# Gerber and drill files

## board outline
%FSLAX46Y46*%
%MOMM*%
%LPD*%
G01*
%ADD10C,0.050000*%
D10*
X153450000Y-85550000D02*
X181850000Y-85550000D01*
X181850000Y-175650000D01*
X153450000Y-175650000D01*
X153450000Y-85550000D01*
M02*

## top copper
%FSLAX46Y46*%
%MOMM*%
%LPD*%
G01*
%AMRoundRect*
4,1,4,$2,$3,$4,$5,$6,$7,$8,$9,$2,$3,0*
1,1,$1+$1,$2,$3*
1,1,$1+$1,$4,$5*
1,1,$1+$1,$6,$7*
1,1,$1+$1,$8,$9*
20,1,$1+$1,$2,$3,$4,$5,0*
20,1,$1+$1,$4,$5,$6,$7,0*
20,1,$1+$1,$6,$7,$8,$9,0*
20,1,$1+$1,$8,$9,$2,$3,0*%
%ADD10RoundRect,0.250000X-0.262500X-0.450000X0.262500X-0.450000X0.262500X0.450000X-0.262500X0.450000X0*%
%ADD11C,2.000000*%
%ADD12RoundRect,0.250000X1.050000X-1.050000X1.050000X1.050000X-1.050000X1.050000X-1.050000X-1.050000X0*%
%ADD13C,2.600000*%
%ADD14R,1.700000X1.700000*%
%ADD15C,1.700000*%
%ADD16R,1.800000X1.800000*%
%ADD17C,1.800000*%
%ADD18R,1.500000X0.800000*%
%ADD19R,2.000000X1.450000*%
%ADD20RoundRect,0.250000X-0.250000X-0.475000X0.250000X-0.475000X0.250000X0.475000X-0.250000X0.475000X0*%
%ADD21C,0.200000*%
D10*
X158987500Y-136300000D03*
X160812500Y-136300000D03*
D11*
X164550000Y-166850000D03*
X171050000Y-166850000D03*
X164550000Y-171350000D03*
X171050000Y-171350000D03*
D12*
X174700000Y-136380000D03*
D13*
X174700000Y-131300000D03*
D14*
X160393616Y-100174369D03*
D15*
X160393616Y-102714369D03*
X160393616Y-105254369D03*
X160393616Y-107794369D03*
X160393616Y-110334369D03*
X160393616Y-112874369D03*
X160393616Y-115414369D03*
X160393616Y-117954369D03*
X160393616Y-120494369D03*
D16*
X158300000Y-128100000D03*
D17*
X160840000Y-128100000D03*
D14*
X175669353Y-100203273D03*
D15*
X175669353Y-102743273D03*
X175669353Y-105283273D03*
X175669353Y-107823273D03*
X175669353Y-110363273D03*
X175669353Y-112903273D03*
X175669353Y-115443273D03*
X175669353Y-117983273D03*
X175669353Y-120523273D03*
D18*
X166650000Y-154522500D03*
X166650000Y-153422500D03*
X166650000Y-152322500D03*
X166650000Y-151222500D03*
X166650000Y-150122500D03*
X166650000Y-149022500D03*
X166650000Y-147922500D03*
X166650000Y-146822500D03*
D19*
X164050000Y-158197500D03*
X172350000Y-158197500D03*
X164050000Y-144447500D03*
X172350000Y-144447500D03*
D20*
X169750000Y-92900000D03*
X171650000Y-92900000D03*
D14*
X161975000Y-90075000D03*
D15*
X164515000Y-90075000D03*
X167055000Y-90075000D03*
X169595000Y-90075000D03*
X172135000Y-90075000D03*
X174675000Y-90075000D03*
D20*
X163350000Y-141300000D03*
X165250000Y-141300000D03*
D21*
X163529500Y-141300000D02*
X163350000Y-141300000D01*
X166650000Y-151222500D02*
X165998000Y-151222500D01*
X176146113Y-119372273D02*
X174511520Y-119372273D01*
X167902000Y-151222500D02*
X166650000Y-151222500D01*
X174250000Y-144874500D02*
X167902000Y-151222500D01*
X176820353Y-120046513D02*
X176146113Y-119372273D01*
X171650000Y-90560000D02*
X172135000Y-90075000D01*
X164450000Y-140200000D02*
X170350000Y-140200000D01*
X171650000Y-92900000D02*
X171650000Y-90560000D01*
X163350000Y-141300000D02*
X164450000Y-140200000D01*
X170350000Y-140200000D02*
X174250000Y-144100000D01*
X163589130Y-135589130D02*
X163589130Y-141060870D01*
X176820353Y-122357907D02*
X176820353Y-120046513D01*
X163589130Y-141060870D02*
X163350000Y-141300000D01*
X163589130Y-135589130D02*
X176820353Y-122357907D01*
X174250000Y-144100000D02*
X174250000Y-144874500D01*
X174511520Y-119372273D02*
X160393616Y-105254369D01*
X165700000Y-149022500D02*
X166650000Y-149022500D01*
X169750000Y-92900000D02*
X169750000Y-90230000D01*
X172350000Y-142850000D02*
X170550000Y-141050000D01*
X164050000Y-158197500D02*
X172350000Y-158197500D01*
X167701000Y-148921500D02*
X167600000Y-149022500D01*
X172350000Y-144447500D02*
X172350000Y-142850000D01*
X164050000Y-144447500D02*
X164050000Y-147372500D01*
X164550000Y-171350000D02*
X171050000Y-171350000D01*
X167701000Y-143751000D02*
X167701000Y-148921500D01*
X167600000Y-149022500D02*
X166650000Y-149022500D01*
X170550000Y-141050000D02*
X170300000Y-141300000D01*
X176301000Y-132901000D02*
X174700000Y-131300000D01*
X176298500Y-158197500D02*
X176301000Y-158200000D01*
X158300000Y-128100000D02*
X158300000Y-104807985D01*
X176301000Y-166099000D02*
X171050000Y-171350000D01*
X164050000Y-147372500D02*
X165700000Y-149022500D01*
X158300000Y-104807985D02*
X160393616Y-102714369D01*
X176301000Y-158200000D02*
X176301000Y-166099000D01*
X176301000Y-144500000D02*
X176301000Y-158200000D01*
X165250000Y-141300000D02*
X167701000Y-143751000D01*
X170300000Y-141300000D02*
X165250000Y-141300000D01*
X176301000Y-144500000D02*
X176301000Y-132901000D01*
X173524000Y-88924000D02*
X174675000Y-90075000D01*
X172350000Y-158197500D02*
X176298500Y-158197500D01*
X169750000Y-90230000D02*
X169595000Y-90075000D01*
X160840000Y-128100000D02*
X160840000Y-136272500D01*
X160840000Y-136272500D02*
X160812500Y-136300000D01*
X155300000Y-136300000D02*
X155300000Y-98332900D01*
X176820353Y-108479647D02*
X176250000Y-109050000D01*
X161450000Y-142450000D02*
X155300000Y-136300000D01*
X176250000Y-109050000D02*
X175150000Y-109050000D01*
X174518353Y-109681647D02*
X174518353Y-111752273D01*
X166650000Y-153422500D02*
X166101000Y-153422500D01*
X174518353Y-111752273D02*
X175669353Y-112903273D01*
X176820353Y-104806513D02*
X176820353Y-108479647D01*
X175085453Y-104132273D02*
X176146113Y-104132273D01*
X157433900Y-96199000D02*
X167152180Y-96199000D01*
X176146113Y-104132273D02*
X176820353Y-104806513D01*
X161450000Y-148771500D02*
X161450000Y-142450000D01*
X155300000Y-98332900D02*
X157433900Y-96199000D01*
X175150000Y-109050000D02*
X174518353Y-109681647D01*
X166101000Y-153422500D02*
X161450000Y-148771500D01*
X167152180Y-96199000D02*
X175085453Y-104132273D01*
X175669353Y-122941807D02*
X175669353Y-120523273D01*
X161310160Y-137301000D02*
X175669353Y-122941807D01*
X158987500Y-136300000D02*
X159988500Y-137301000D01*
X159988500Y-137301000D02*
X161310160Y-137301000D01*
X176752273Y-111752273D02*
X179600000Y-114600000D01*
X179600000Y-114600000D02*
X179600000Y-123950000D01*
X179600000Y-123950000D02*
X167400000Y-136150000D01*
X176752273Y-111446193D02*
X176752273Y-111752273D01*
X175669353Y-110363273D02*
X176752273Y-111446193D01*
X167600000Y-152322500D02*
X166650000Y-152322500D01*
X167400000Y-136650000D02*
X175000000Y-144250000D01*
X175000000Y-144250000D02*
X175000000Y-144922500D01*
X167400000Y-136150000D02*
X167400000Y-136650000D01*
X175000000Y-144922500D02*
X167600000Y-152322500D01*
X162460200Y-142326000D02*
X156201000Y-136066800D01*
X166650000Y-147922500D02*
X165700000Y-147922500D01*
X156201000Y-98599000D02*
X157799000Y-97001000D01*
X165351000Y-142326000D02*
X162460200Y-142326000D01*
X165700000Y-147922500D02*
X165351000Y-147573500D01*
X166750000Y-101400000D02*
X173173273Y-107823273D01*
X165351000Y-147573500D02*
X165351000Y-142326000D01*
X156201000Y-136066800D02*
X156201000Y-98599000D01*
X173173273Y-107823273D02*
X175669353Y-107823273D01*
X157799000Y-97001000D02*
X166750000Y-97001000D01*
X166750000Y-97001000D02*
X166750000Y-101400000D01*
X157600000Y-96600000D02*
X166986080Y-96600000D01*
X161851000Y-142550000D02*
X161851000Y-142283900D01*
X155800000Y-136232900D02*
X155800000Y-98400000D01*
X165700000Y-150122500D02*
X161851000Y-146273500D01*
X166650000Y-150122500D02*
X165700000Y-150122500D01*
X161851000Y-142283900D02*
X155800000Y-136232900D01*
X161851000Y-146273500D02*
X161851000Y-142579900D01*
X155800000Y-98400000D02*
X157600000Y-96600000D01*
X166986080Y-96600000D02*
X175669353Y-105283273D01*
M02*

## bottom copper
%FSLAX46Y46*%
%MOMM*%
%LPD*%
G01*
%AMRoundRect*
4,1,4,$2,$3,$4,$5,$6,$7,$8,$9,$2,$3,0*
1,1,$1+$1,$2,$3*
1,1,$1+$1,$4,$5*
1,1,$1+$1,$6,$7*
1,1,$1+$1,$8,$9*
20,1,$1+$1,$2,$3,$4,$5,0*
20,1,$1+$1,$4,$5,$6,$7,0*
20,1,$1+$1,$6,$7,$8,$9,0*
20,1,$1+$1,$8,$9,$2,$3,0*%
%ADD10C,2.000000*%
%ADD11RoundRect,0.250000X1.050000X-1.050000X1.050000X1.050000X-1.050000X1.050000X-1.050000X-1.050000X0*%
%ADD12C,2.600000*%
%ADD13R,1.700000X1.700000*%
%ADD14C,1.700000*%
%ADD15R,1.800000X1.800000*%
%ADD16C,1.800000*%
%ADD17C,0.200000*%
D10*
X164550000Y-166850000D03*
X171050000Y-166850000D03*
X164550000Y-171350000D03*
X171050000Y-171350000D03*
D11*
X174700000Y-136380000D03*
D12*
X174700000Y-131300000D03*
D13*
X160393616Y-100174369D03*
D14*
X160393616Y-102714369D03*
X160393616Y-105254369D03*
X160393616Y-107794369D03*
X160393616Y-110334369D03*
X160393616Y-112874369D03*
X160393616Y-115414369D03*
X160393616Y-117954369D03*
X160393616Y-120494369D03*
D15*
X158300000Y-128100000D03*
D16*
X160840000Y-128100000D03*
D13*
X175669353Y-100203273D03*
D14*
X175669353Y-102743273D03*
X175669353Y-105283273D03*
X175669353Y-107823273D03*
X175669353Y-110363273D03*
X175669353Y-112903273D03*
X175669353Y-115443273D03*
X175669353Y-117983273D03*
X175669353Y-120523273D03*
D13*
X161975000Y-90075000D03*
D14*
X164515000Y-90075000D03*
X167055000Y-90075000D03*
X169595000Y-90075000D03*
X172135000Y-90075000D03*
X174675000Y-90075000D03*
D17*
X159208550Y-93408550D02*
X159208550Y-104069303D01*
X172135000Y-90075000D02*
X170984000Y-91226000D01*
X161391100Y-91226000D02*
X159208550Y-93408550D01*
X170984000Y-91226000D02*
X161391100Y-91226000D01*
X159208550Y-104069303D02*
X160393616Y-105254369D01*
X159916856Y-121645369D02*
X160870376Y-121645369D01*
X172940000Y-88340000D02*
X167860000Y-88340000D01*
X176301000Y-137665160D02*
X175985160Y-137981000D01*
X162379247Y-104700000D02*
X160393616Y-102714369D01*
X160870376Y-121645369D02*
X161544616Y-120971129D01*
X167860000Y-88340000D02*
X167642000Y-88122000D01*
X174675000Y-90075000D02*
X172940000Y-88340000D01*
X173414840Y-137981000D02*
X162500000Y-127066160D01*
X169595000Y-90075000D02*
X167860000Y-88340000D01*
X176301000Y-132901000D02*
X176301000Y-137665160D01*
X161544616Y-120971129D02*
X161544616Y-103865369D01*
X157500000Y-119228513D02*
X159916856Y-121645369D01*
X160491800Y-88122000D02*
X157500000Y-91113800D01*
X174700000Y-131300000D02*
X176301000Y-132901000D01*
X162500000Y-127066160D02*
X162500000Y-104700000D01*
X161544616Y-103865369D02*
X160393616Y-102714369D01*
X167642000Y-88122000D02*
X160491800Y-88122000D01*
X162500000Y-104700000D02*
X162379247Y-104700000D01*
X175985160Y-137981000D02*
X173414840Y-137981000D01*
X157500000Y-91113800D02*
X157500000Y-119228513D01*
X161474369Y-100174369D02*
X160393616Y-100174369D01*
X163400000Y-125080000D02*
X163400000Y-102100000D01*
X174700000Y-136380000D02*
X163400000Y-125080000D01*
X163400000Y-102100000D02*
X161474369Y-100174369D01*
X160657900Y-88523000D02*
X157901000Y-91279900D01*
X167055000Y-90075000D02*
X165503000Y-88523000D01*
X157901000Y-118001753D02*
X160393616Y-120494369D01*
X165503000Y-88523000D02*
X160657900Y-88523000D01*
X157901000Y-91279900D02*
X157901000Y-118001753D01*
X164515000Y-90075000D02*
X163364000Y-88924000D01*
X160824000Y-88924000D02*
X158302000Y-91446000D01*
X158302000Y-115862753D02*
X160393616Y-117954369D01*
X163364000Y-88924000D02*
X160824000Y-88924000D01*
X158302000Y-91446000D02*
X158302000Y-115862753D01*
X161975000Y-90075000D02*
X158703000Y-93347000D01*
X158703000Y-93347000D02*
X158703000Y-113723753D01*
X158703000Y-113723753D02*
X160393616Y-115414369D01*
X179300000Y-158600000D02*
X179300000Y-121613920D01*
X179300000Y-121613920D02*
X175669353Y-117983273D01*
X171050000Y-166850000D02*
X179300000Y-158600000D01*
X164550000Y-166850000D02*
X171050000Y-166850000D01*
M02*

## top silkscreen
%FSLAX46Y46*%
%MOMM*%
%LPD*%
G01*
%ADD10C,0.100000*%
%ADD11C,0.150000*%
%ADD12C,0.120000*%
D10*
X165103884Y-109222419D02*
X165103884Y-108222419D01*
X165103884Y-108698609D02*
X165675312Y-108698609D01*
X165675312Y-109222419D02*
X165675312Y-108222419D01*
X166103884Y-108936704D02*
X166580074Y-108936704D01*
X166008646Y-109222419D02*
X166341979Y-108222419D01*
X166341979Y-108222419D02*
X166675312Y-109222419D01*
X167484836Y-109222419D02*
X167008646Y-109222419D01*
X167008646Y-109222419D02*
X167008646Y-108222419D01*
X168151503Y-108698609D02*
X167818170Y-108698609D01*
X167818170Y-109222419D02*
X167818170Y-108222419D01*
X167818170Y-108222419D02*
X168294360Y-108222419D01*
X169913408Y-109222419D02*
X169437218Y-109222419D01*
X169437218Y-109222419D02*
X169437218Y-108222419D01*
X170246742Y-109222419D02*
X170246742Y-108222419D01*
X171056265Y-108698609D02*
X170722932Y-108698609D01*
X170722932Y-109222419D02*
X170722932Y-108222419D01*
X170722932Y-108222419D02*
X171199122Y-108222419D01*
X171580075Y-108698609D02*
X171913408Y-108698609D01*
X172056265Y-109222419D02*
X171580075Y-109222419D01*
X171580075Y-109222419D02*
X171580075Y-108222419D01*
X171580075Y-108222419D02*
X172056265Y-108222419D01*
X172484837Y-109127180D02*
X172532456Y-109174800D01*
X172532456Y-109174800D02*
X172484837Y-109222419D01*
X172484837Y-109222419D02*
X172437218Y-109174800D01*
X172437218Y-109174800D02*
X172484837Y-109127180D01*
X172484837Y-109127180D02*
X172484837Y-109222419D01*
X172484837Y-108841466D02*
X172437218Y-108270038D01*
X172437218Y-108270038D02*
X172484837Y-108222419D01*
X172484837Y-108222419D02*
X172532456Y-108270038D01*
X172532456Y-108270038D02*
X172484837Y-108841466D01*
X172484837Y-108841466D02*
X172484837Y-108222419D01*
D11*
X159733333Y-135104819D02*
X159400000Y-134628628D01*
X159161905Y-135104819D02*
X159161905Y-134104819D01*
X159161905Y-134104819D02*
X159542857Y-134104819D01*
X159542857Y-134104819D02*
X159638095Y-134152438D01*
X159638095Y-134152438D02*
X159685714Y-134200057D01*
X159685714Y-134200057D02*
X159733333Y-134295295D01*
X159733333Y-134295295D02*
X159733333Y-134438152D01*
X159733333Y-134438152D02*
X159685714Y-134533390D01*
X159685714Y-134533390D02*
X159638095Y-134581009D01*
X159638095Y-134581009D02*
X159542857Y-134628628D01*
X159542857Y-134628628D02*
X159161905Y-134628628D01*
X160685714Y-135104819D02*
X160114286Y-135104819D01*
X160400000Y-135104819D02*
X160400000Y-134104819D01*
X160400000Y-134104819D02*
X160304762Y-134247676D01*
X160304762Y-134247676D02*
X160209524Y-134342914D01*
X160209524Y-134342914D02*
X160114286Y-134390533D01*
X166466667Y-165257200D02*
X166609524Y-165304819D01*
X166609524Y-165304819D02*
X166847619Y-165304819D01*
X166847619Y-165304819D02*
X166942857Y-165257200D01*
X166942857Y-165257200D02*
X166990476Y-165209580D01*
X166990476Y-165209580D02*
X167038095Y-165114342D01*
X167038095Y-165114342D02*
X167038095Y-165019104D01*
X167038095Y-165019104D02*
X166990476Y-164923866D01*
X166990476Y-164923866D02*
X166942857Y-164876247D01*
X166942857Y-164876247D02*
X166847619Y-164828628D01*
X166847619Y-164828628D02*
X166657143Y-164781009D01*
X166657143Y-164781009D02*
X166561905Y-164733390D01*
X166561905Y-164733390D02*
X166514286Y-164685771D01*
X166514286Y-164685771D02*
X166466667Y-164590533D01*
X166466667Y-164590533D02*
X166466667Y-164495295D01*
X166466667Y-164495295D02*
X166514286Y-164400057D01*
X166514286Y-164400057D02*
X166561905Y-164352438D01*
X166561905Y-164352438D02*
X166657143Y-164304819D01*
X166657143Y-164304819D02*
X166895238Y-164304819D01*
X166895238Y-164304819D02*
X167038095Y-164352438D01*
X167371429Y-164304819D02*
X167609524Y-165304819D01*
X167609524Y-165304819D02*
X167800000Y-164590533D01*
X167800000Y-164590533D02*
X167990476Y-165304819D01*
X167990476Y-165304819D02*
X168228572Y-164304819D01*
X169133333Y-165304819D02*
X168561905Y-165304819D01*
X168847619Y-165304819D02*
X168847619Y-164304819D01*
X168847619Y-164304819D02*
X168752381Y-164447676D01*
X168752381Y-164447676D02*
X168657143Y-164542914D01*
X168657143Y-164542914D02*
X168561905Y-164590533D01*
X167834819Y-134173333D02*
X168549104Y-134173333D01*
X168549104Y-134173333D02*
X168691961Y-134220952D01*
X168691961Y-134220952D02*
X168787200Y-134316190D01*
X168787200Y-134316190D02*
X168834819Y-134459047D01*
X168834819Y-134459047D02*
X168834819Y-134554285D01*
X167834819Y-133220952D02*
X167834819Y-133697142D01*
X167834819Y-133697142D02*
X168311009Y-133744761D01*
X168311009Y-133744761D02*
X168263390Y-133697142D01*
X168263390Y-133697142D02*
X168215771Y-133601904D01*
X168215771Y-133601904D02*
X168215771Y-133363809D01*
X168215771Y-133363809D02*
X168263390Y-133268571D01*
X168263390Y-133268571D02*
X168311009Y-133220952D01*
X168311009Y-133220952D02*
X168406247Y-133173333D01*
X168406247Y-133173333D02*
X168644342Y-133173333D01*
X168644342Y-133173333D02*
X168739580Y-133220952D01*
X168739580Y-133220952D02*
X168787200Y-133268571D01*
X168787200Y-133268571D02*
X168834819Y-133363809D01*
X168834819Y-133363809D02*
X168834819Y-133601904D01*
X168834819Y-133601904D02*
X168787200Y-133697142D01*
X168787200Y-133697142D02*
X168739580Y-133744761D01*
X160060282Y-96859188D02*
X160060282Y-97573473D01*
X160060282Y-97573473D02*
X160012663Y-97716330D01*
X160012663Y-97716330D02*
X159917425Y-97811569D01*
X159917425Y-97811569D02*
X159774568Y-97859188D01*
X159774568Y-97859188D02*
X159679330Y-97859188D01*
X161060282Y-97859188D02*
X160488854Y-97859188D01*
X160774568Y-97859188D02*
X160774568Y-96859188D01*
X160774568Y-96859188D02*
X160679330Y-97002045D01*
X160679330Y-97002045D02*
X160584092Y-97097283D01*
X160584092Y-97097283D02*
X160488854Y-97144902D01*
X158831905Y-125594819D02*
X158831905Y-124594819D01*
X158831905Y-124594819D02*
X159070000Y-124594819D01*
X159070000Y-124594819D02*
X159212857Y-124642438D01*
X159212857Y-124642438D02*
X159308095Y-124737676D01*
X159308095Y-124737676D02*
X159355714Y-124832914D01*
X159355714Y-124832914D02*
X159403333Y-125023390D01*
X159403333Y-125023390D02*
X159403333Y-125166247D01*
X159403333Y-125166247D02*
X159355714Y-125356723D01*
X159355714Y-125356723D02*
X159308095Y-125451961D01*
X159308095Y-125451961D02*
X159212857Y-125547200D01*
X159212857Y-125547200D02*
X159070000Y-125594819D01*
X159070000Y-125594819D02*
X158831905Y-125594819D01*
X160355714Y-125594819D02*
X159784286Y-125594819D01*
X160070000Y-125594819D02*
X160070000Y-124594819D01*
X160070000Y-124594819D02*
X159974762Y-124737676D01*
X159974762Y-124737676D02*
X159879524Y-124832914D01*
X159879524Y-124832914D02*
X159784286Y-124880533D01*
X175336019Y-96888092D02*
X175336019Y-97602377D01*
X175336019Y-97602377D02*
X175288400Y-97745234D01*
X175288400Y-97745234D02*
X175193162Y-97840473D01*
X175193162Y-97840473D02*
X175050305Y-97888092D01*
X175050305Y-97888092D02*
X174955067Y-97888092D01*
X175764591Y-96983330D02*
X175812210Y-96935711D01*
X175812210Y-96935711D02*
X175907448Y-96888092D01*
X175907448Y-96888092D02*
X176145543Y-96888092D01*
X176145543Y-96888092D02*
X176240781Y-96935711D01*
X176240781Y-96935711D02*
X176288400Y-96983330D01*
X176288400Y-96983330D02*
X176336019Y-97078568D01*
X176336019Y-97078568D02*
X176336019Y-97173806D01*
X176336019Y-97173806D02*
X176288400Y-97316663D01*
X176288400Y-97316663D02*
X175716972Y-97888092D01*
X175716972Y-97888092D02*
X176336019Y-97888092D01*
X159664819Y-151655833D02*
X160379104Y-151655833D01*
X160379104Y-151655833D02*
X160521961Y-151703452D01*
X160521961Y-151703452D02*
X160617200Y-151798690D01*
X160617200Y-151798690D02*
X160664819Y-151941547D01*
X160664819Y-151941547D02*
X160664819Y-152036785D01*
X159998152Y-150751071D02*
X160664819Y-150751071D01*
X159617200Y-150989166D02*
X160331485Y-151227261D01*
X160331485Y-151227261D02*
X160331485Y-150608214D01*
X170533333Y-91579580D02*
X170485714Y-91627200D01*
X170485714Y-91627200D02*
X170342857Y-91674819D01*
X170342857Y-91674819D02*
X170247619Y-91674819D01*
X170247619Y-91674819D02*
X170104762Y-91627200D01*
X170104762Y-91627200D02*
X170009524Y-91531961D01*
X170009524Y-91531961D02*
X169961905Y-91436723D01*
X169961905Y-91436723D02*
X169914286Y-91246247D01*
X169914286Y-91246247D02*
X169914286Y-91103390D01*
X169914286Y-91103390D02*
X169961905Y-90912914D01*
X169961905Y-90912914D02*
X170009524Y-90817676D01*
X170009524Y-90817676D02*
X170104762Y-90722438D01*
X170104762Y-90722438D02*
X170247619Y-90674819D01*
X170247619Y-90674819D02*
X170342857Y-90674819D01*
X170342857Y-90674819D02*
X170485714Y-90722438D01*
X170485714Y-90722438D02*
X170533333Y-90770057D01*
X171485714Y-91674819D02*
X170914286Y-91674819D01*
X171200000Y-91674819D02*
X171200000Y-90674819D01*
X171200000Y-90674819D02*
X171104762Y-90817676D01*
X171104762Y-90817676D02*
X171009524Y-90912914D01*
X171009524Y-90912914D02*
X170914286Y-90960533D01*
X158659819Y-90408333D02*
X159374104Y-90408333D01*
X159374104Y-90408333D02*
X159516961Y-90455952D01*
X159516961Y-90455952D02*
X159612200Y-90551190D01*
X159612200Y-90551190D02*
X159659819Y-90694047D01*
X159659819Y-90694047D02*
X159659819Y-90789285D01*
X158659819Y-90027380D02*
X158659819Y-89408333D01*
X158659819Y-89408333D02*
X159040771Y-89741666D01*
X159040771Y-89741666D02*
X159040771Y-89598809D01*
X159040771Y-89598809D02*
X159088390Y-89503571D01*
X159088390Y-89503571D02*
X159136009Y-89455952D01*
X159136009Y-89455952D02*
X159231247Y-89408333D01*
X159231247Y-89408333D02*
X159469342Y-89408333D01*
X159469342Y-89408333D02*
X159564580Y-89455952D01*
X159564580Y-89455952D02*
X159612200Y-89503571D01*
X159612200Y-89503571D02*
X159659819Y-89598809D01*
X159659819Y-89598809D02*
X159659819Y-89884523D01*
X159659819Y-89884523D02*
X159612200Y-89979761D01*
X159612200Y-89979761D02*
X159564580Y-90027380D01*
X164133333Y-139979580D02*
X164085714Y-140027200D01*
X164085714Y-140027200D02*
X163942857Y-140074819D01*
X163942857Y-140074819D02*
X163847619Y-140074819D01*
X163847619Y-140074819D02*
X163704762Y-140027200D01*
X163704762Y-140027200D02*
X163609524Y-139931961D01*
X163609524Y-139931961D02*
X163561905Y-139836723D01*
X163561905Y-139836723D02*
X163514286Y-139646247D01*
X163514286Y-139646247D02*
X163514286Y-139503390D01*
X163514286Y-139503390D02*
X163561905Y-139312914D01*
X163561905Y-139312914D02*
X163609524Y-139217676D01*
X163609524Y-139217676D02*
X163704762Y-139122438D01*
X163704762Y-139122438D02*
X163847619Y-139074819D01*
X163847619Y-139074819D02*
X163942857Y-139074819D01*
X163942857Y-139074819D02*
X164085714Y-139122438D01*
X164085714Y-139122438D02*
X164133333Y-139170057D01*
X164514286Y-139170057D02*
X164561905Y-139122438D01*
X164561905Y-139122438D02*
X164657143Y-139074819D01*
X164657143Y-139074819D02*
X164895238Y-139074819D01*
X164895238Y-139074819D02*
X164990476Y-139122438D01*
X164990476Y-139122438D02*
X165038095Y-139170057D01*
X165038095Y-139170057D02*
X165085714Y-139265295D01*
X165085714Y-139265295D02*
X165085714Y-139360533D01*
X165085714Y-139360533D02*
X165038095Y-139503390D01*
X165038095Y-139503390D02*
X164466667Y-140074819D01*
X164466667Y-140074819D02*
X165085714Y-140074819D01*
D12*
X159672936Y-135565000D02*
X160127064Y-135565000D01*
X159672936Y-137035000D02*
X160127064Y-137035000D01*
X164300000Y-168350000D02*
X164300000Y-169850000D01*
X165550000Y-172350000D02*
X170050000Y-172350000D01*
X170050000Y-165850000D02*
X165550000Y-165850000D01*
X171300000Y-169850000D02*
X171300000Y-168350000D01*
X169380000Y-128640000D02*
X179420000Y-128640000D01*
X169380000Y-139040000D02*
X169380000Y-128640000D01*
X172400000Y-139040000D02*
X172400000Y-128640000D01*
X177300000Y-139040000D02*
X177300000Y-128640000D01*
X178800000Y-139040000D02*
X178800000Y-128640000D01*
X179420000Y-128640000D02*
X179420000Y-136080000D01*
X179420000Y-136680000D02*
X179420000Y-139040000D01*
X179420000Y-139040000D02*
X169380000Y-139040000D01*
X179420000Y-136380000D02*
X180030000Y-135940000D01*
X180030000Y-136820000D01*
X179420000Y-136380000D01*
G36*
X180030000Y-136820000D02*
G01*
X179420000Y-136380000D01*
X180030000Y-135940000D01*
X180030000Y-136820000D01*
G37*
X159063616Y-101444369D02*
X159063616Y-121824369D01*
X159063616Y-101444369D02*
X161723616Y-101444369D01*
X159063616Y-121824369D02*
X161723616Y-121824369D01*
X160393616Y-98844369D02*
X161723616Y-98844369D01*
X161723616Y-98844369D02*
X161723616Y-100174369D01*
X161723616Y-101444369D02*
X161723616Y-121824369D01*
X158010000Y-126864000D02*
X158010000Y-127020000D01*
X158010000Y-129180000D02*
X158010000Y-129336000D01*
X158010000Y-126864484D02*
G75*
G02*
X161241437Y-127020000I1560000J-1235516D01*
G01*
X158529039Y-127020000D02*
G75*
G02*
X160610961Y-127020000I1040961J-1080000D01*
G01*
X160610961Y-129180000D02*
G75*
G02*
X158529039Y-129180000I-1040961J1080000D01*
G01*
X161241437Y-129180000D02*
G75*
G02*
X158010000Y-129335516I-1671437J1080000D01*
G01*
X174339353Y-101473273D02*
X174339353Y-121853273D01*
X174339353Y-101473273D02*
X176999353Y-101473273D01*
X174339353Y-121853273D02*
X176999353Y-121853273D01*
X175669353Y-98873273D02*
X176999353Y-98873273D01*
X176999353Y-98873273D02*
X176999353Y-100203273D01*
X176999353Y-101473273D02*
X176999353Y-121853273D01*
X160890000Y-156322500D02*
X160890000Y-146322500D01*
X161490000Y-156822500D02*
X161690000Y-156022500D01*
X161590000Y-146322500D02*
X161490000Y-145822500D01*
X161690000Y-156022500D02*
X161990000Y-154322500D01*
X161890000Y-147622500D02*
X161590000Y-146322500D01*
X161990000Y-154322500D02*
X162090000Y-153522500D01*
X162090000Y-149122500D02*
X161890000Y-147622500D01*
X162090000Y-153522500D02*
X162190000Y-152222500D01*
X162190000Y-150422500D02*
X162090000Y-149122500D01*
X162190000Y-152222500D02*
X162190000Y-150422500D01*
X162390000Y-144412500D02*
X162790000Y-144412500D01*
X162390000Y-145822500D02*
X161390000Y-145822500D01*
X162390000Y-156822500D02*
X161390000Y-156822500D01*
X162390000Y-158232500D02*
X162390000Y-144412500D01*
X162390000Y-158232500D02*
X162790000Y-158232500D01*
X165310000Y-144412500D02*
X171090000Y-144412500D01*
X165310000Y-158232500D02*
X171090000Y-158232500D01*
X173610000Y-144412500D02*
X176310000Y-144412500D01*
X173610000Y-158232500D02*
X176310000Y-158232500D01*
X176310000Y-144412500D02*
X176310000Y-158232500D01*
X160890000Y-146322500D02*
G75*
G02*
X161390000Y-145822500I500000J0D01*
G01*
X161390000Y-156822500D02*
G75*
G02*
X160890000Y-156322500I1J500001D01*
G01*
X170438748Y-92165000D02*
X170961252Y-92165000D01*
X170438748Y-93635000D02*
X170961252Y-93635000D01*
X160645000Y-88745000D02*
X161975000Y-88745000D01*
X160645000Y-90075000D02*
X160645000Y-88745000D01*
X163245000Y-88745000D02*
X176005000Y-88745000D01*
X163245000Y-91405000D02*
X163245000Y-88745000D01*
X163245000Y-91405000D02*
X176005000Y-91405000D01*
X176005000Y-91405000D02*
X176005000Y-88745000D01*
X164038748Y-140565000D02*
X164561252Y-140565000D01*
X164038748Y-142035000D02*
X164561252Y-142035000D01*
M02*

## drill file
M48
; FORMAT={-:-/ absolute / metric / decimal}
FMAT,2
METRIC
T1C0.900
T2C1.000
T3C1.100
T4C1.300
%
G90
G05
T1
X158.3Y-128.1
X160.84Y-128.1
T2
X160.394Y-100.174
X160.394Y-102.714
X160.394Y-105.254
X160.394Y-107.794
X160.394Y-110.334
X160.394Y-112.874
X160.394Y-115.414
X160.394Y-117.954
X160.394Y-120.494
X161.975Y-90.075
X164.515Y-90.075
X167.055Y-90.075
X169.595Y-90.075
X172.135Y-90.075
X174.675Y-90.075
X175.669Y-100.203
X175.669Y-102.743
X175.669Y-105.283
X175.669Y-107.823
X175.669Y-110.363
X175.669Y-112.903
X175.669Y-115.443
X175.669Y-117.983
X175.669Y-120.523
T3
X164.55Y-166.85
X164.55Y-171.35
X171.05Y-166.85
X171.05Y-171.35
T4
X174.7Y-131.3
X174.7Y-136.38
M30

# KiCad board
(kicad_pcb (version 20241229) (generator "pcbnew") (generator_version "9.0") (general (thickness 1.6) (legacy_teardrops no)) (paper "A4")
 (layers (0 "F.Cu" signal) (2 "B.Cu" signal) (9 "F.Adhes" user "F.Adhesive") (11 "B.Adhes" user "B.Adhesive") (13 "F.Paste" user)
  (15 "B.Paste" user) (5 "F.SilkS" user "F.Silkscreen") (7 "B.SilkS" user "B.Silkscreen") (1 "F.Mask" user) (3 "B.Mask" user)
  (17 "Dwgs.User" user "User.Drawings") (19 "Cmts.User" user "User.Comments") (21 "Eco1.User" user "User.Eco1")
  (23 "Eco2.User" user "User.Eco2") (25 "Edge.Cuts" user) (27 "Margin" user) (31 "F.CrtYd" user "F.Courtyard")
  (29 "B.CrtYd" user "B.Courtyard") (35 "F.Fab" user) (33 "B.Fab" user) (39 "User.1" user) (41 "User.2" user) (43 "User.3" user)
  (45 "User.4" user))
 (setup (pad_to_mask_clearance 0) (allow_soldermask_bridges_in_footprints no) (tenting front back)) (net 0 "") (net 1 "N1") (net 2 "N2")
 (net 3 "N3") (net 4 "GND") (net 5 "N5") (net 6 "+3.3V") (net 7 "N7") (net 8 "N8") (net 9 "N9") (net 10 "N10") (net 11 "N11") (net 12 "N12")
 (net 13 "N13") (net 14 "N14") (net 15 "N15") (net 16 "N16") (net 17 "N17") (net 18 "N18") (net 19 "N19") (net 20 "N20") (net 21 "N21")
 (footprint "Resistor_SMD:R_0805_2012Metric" (layer "F.Cu") (at 159.9 136.3)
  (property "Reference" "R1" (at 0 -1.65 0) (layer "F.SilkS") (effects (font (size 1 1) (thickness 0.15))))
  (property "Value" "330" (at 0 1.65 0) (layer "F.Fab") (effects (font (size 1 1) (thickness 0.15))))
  (fp_line (start -0.227064 -0.735) (end 0.227064 -0.735) (stroke (width 0.12) (type solid)) (layer "F.SilkS"))
  (fp_line (start -0.227064 0.735) (end 0.227064 0.735) (stroke (width 0.12) (type solid)) (layer "F.SilkS"))
  (pad "1" smd roundrect (at -0.9125 0) (size 1.025 1.4) (layers "F.Cu" "F.Mask" "F.Paste") (roundrect_rratio 0.243902) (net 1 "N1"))
  (pad "2" smd roundrect (at 0.9125 0) (size 1.025 1.4) (layers "F.Cu" "F.Mask" "F.Paste") (roundrect_rratio 0.243902) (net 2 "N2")))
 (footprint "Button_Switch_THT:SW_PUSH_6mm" (layer "F.Cu") (at 164.55 166.85)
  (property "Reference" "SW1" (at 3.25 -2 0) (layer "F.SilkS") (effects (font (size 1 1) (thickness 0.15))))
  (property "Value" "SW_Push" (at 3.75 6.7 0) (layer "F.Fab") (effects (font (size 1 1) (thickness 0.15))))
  (fp_line (start -0.25 1.5) (end -0.25 3) (stroke (width 0.12) (type solid)) (layer "F.SilkS"))
  (fp_line (start 1 5.5) (end 5.5 5.5) (stroke (width 0.12) (type solid)) (layer "F.SilkS"))
  (fp_line (start 5.5 -1) (end 1 -1) (stroke (width 0.12) (type solid)) (layer "F.SilkS"))
  (fp_line (start 6.75 3) (end 6.75 1.5) (stroke (width 0.12) (type solid)) (layer "F.SilkS"))
  (pad "1" thru_hole circle (at 0 0 90) (size 2 2) (drill 1.1) (layers "*.Cu" "*.Mask") (remove_unused_layers no) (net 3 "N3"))
  (pad "1" thru_hole circle (at 6.5 0 90) (size 2 2) (drill 1.1) (layers "*.Cu" "*.Mask") (remove_unused_layers no) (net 3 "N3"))
  (pad "2" thru_hole circle (at 0 4.5 90) (size 2 2) (drill 1.1) (layers "*.Cu" "*.Mask") (remove_unused_layers no) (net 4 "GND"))
  (pad "2" thru_hole circle (at 6.5 4.5 90) (size 2 2) (drill 1.1) (layers "*.Cu" "*.Mask") (remove_unused_layers no) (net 4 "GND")))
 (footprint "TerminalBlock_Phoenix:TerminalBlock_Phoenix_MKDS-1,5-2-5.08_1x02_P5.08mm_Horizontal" (layer "F.Cu") (at 174.7 136.38 90)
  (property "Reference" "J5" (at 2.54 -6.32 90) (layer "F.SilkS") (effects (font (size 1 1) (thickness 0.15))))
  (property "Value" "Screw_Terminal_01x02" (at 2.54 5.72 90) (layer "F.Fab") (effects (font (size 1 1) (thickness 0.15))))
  (fp_line (start 7.74 -5.32) (end 7.74 4.72) (stroke (width 0.12) (type solid)) (layer "F.SilkS"))
  (fp_line (start -2.66 -5.32) (end 7.74 -5.32) (stroke (width 0.12) (type solid)) (layer "F.SilkS"))
  (fp_line (start -2.66 -2.3) (end 7.74 -2.3) (stroke (width 0.12) (type solid)) (layer "F.SilkS"))
  (fp_line (start -2.66 2.6) (end 7.74 2.6) (stroke (width 0.12) (type solid)) (layer "F.SilkS"))
  (fp_line (start -2.66 4.1) (end 7.74 4.1) (stroke (width 0.12) (type solid)) (layer "F.SilkS"))
  (fp_line (start 7.74 4.72) (end 0.3 4.72) (stroke (width 0.12) (type solid)) (layer "F.SilkS"))
  (fp_line (start -0.3 4.72) (end -2.66 4.72) (stroke (width 0.12) (type solid)) (layer "F.SilkS"))
  (fp_line (start -2.66 4.72) (end -2.66 -5.32) (stroke (width 0.12) (type solid)) (layer "F.SilkS"))
  (fp_poly (pts (xy 0 4.72) (xy 0.44 5.33) (xy -0.44 5.33)) (stroke (width 0.12) (type solid)) (fill yes) (layer "F.SilkS"))
  (pad "1" thru_hole roundrect (at 0 0 90) (size 2.6 2.6) (drill 1.3) (layers "*.Cu" "*.Mask") (remove_unused_layers no)
   (roundrect_rratio 0.096154) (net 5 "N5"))
  (pad "2" thru_hole circle (at 5.08 0 90) (size 2.6 2.6) (drill 1.3) (layers "*.Cu" "*.Mask") (remove_unused_layers no) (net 4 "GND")))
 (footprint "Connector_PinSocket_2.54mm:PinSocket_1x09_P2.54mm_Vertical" (layer "F.Cu") (at 160.393616 100.174369)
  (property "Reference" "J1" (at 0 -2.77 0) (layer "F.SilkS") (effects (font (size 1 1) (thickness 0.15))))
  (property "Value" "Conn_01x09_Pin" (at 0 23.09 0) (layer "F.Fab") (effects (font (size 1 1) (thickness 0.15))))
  (fp_line (start -1.33 1.27) (end -1.33 21.65) (stroke (width 0.12) (type solid)) (layer "F.SilkS"))
  (fp_line (start -1.33 1.27) (end 1.33 1.27) (stroke (width 0.12) (type solid)) (layer "F.SilkS"))
  (fp_line (start -1.33 21.65) (end 1.33 21.65) (stroke (width 0.12) (type solid)) (layer "F.SilkS"))
  (fp_line (start 0 -1.33) (end 1.33 -1.33) (stroke (width 0.12) (type solid)) (layer "F.SilkS"))
  (fp_line (start 1.33 -1.33) (end 1.33 0) (stroke (width 0.12) (type solid)) (layer "F.SilkS"))
  (fp_line (start 1.33 1.27) (end 1.33 21.65) (stroke (width 0.12) (type solid)) (layer "F.SilkS"))
  (pad "1" thru_hole rect (at 0 0) (size 1.7 1.7) (drill 1) (layers "*.Cu" "*.Mask") (remove_unused_layers no) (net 5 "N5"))
  (pad "2" thru_hole circle (at 0 2.54) (size 1.7 1.7) (drill 1) (layers "*.Cu" "*.Mask") (remove_unused_layers no) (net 4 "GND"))
  (pad "3" thru_hole circle (at 0 5.08) (size 1.7 1.7) (drill 1) (layers "*.Cu" "*.Mask") (remove_unused_layers no) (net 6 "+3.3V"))
  (pad "4" thru_hole circle (at 0 7.62) (size 1.7 1.7) (drill 1) (layers "*.Cu" "*.Mask") (remove_unused_layers no) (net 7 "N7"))
  (pad "5" thru_hole circle (at 0 10.16) (size 1.7 1.7) (drill 1) (layers "*.Cu" "*.Mask") (remove_unused_layers no) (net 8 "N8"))
  (pad "6" thru_hole circle (at 0 12.7) (size 1.7 1.7) (drill 1) (layers "*.Cu" "*.Mask") (remove_unused_layers no) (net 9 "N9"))
  (pad "7" thru_hole circle (at 0 15.24) (size 1.7 1.7) (drill 1) (layers "*.Cu" "*.Mask") (remove_unused_layers no) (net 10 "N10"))
  (pad "8" thru_hole circle (at 0 17.78) (size 1.7 1.7) (drill 1) (layers "*.Cu" "*.Mask") (remove_unused_layers no) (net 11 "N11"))
  (pad "9" thru_hole circle (at 0 20.32) (size 1.7 1.7) (drill 1) (layers "*.Cu" "*.Mask") (remove_unused_layers no) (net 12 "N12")))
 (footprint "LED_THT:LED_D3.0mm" (layer "F.Cu") (at 158.3 128.1)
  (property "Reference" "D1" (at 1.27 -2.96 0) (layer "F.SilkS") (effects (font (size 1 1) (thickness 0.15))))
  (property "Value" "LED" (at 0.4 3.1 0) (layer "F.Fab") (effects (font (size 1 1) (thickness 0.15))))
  (fp_line (start -0.29 -1.236) (end -0.29 -1.08) (stroke (width 0.12) (type solid)) (layer "F.SilkS"))
  (fp_line (start -0.29 1.08) (end -0.29 1.236) (stroke (width 0.12) (type solid)) (layer "F.SilkS"))
  (fp_arc (start -0.29 -1.235516) (mid 1.36566 -1.987699) (end 2.941437 -1.08) (stroke (width 0.12) (type solid)) (layer "F.SilkS"))
  (fp_arc (start 0.229039 -1.08) (mid 1.27 -1.5) (end 2.310961 -1.08) (stroke (width 0.12) (type solid)) (layer "F.SilkS"))
  (fp_arc (start 2.310961 1.08) (mid 1.27 1.5) (end 0.229039 1.08) (stroke (width 0.12) (type solid)) (layer "F.SilkS"))
  (fp_arc (start 2.941437 1.08) (mid 1.36566 1.987699) (end -0.29 1.235516) (stroke (width 0.12) (type solid)) (layer "F.SilkS"))
  (pad "1" thru_hole rect (at 0 0) (size 1.8 1.8) (drill 0.9) (layers "*.Cu" "*.Mask") (remove_unused_layers no) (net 4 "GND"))
  (pad "2" thru_hole circle (at 2.54 0) (size 1.8 1.8) (drill 0.9) (layers "*.Cu" "*.Mask") (remove_unused_layers no) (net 2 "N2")))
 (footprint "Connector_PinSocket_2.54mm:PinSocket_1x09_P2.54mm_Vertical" (layer "F.Cu") (at 175.669353 100.203273)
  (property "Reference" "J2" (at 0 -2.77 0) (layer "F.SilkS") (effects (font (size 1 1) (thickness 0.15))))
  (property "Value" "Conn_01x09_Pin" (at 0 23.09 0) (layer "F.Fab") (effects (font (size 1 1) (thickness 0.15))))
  (fp_line (start -1.33 1.27) (end -1.33 21.65) (stroke (width 0.12) (type solid)) (layer "F.SilkS"))
  (fp_line (start -1.33 1.27) (end 1.33 1.27) (stroke (width 0.12) (type solid)) (layer "F.SilkS"))
  (fp_line (start -1.33 21.65) (end 1.33 21.65) (stroke (width 0.12) (type solid)) (layer "F.SilkS"))
  (fp_line (start 0 -1.33) (end 1.33 -1.33) (stroke (width 0.12) (type solid)) (layer "F.SilkS"))
  (fp_line (start 1.33 -1.33) (end 1.33 0) (stroke (width 0.12) (type solid)) (layer "F.SilkS"))
  (fp_line (start 1.33 1.27) (end 1.33 21.65) (stroke (width 0.12) (type solid)) (layer "F.SilkS"))
  (pad "1" thru_hole rect (at 0 0) (size 1.7 1.7) (drill 1) (layers "*.Cu" "*.Mask") (remove_unused_layers no) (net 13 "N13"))
  (pad "2" thru_hole circle (at 0 2.54) (size 1.7 1.7) (drill 1) (layers "*.Cu" "*.Mask") (remove_unused_layers no) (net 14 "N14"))
  (pad "3" thru_hole circle (at 0 5.08) (size 1.7 1.7) (drill 1) (layers "*.Cu" "*.Mask") (remove_unused_layers no) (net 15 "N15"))
  (pad "4" thru_hole circle (at 0 7.62) (size 1.7 1.7) (drill 1) (layers "*.Cu" "*.Mask") (remove_unused_layers no) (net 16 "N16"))
  (pad "5" thru_hole circle (at 0 10.16) (size 1.7 1.7) (drill 1) (layers "*.Cu" "*.Mask") (remove_unused_layers no) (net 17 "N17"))
  (pad "6" thru_hole circle (at 0 12.7) (size 1.7 1.7) (drill 1) (layers "*.Cu" "*.Mask") (remove_unused_layers no) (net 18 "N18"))
  (pad "7" thru_hole circle (at 0 15.24) (size 1.7 1.7) (drill 1) (layers "*.Cu" "*.Mask") (remove_unused_layers no) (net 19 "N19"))
  (pad "8" thru_hole circle (at 0 17.78) (size 1.7 1.7) (drill 1) (layers "*.Cu" "*.Mask") (remove_unused_layers no) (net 3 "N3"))
  (pad "9" thru_hole circle (at 0 20.32) (size 1.7 1.7) (drill 1) (layers "*.Cu" "*.Mask") (remove_unused_layers no) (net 1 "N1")))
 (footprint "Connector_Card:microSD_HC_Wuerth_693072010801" (layer "F.Cu") (at 168.2 151.3225 90)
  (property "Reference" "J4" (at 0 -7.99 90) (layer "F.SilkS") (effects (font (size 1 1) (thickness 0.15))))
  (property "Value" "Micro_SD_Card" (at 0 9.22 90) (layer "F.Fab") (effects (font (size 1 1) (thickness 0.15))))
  (fp_line (start -5 -7.31) (end 5 -7.31) (stroke (width 0.12) (type solid)) (layer "F.SilkS"))
  (fp_line (start -5.5 -6.71) (end -4.7 -6.51) (stroke (width 0.12) (type solid)) (layer "F.SilkS"))
  (fp_line (start 5 -6.61) (end 5.5 -6.71) (stroke (width 0.12) (type solid)) (layer "F.SilkS"))
  (fp_line (start -4.7 -6.51) (end -3 -6.21) (stroke (width 0.12) (type solid)) (layer "F.SilkS"))
  (fp_line (start 3.7 -6.31) (end 5 -6.61) (stroke (width 0.12) (type solid)) (layer "F.SilkS"))
  (fp_line (start -3 -6.21) (end -2.2 -6.11) (stroke (width 0.12) (type solid)) (layer "F.SilkS"))
  (fp_line (start 2.2 -6.11) (end 3.7 -6.31) (stroke (width 0.12) (type solid)) (layer "F.SilkS"))
  (fp_line (start -2.2 -6.11) (end -0.9 -6.01) (stroke (width 0.12) (type solid)) (layer "F.SilkS"))
  (fp_line (start 0.9 -6.01) (end 2.2 -6.11) (stroke (width 0.12) (type solid)) (layer "F.SilkS"))
  (fp_line (start -0.9 -6.01) (end 0.9 -6.01) (stroke (width 0.12) (type solid)) (layer "F.SilkS"))
  (fp_line (start 6.91 -5.81) (end 6.91 -5.41) (stroke (width 0.12) (type solid)) (layer "F.SilkS"))
  (fp_line (start 5.5 -5.81) (end 5.5 -6.81) (stroke (width 0.12) (type solid)) (layer "F.SilkS"))
  (fp_line (start -5.5 -5.81) (end -5.5 -6.81) (stroke (width 0.12) (type solid)) (layer "F.SilkS"))
  (fp_line (start -6.91 -5.81) (end 6.91 -5.81) (stroke (width 0.12) (type solid)) (layer "F.SilkS"))
  (fp_line (start -6.91 -5.81) (end -6.91 -5.41) (stroke (width 0.12) (type solid)) (layer "F.SilkS"))
  (fp_line (start 6.91 -2.89) (end 6.91 2.89) (stroke (width 0.12) (type solid)) (layer "F.SilkS"))
  (fp_line (start -6.91 -2.89) (end -6.91 2.89) (stroke (width 0.12) (type solid)) (layer "F.SilkS"))
  (fp_line (start 6.91 5.41) (end 6.91 8.11) (stroke (width 0.12) (type solid)) (layer "F.SilkS"))
  (fp_line (start -6.91 5.41) (end -6.91 8.11) (stroke (width 0.12) (type solid)) (layer "F.SilkS"))
  (fp_line (start 6.91 8.11) (end -6.91 8.11) (stroke (width 0.12) (type solid)) (layer "F.SilkS"))
  (fp_arc (start 5 -7.31) (mid 5.353553 -7.163553) (end 5.5 -6.81) (stroke (width 0.12) (type solid)) (layer "F.SilkS"))
  (fp_arc (start -5.5 -6.81) (mid -5.353553 -7.163553) (end -5 -7.31) (stroke (width 0.12) (type solid)) (layer "F.SilkS"))
  (pad "1" smd rect (at -3.2 -1.55 90) (size 0.8 1.5) (layers "F.Cu" "F.Mask" "F.Paste") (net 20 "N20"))
  (pad "2" smd rect (at -2.1 -1.55 90) (size 0.8 1.5) (layers "F.Cu" "F.Mask" "F.Paste") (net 18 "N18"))
  (pad "3" smd rect (at -1 -1.55 90) (size 0.8 1.5) (layers "F.Cu" "F.Mask" "F.Paste") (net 17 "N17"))
  (pad "4" smd rect (at 0.1 -1.55 90) (size 0.8 1.5) (layers "F.Cu" "F.Mask" "F.Paste") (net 6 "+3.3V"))
  (pad "5" smd rect (at 1.2 -1.55 90) (size 0.8 1.5) (layers "F.Cu" "F.Mask" "F.Paste") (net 15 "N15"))
  (pad "6" smd rect (at 2.3 -1.55 90) (size 0.8 1.5) (layers "F.Cu" "F.Mask" "F.Paste") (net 4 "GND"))
  (pad "7" smd rect (at 3.4 -1.55 90) (size 0.8 1.5) (layers "F.Cu" "F.Mask" "F.Paste") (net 16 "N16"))
  (pad "8" smd rect (at 4.5 -1.55 90) (size 0.8 1.5) (layers "F.Cu" "F.Mask" "F.Paste") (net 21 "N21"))
  (pad "9" smd rect (at -6.875 -4.15 90) (size 1.45 2) (layers "F.Cu" "F.Mask" "F.Paste") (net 4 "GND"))
  (pad "9" smd rect (at -6.875 4.15 90) (size 1.45 2) (layers "F.Cu" "F.Mask" "F.Paste") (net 4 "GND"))
  (pad "9" smd rect (at 6.875 -4.15 90) (size 1.45 2) (layers "F.Cu" "F.Mask" "F.Paste") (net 4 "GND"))
  (pad "9" smd rect (at 6.875 4.15 90) (size 1.45 2) (layers "F.Cu" "F.Mask" "F.Paste") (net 4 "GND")))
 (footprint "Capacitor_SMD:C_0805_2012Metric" (layer "F.Cu") (at 170.7 92.9)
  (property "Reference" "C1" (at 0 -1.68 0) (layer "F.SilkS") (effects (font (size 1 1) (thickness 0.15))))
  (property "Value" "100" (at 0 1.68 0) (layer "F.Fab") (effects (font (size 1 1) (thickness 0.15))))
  (fp_line (start -0.261252 -0.735) (end 0.261252 -0.735) (stroke (width 0.12) (type solid)) (layer "F.SilkS"))
  (fp_line (start -0.261252 0.735) (end 0.261252 0.735) (stroke (width 0.12) (type solid)) (layer "F.SilkS"))
  (pad "1" smd roundrect (at -0.95 0) (size 1 1.45) (layers "F.Cu" "F.Mask" "F.Paste") (roundrect_rratio 0.25) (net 4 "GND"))
  (pad "2" smd roundrect (at 0.95 0) (size 1 1.45) (layers "F.Cu" "F.Mask" "F.Paste") (roundrect_rratio 0.25) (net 6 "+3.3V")))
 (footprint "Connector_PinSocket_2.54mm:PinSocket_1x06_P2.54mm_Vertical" (layer "F.Cu") (at 161.975 90.075 90)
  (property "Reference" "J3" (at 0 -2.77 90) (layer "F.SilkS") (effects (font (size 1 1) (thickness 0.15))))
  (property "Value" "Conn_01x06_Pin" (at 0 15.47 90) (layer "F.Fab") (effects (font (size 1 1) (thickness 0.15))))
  (fp_line (start 1.33 -1.33) (end 1.33 0) (stroke (width 0.12) (type solid)) (layer "F.SilkS"))
  (fp_line (start 0 -1.33) (end 1.33 -1.33) (stroke (width 0.12) (type solid)) (layer "F.SilkS"))
  (fp_line (start 1.33 1.27) (end 1.33 14.03) (stroke (width 0.12) (type solid)) (layer "F.SilkS"))
  (fp_line (start -1.33 1.27) (end 1.33 1.27) (stroke (width 0.12) (type solid)) (layer "F.SilkS"))
  (fp_line (start -1.33 1.27) (end -1.33 14.03) (stroke (width 0.12) (type solid)) (layer "F.SilkS"))
  (fp_line (start -1.33 14.03) (end 1.33 14.03) (stroke (width 0.12) (type solid)) (layer "F.SilkS"))
  (pad "1" thru_hole rect (at 0 0 90) (size 1.7 1.7) (drill 1) (layers "*.Cu" "*.Mask") (remove_unused_layers no) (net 10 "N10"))
  (pad "2" thru_hole circle (at 0 2.54 90) (size 1.7 1.7) (drill 1) (layers "*.Cu" "*.Mask") (remove_unused_layers no) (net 11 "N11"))
  (pad "3" thru_hole circle (at 0 5.08 90) (size 1.7 1.7) (drill 1) (layers "*.Cu" "*.Mask") (remove_unused_layers no) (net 12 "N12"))
  (pad "4" thru_hole circle (at 0 7.62 90) (size 1.7 1.7) (drill 1) (layers "*.Cu" "*.Mask") (remove_unused_layers no) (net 4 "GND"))
  (pad "5" thru_hole circle (at 0 10.16 90) (size 1.7 1.7) (drill 1) (layers "*.Cu" "*.Mask") (remove_unused_layers no) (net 6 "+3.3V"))
  (pad "6" thru_hole circle (at 0 12.7 90) (size 1.7 1.7) (drill 1) (layers "*.Cu" "*.Mask") (remove_unused_layers no) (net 4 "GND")))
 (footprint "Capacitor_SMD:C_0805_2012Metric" (layer "F.Cu") (at 164.3 141.3)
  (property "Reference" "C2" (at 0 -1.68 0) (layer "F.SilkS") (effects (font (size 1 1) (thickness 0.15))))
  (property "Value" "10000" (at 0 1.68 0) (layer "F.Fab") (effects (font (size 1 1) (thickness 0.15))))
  (fp_line (start -0.261252 -0.735) (end 0.261252 -0.735) (stroke (width 0.12) (type solid)) (layer "F.SilkS"))
  (fp_line (start -0.261252 0.735) (end 0.261252 0.735) (stroke (width 0.12) (type solid)) (layer "F.SilkS"))
  (pad "1" smd roundrect (at -0.95 0) (size 1 1.45) (layers "F.Cu" "F.Mask" "F.Paste") (roundrect_rratio 0.25) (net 6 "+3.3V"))
  (pad "2" smd roundrect (at 0.95 0) (size 1 1.45) (layers "F.Cu" "F.Mask" "F.Paste") (roundrect_rratio 0.25) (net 4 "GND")))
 (gr_rect (start 153.45 85.55) (end 181.85 175.65) (stroke (width 0.05) (type default)) (fill no) (layer "Edge.Cuts"))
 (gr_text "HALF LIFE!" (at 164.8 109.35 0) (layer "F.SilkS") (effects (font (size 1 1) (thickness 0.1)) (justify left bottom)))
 (segment (start 163.5295 141.3) (end 163.35 141.3) (width 0.2) (layer "F.Cu") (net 6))
 (segment (start 166.65 151.2225) (end 165.998 151.2225) (width 0.2) (layer "F.Cu") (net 6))
 (segment (start 176.146113 119.372273) (end 174.51152 119.372273) (width 0.2) (layer "F.Cu") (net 6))
 (segment (start 167.902 151.2225) (end 166.65 151.2225) (width 0.2) (layer "F.Cu") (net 6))
 (segment (start 174.25 144.8745) (end 167.902 151.2225) (width 0.2) (layer "F.Cu") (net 6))
 (segment (start 176.820353 120.046513) (end 176.146113 119.372273) (width 0.2) (layer "F.Cu") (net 6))
 (segment (start 171.65 90.56) (end 172.135 90.075) (width 0.2) (layer "F.Cu") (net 6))
 (segment (start 164.45 140.2) (end 170.35 140.2) (width 0.2) (layer "F.Cu") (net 6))
 (segment (start 171.65 92.9) (end 171.65 90.56) (width 0.2) (layer "F.Cu") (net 6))
 (segment (start 163.35 141.3) (end 164.45 140.2) (width 0.2) (layer "F.Cu") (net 6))
 (segment (start 170.35 140.2) (end 174.25 144.1) (width 0.2) (layer "F.Cu") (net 6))
 (segment (start 163.58913 135.58913) (end 163.58913 141.06087) (width 0.2) (layer "F.Cu") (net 6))
 (segment (start 176.820353 122.357907) (end 176.820353 120.046513) (width 0.2) (layer "F.Cu") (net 6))
 (segment (start 163.58913 141.06087) (end 163.35 141.3) (width 0.2) (layer "F.Cu") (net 6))
 (segment (start 163.58913 135.58913) (end 176.820353 122.357907) (width 0.2) (layer "F.Cu") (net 6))
 (segment (start 174.25 144.1) (end 174.25 144.8745) (width 0.2) (layer "F.Cu") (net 6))
 (segment (start 174.51152 119.372273) (end 160.393616 105.254369) (width 0.2) (layer "F.Cu") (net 6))
 (segment (start 159.20855 93.40855) (end 159.20855 104.069303) (width 0.2) (layer "B.Cu") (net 6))
 (segment (start 172.135 90.075) (end 170.984 91.226) (width 0.2) (layer "B.Cu") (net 6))
 (segment (start 161.3911 91.226) (end 159.20855 93.40855) (width 0.2) (layer "B.Cu") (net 6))
 (segment (start 170.984 91.226) (end 161.3911 91.226) (width 0.2) (layer "B.Cu") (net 6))
 (segment (start 159.20855 104.069303) (end 160.393616 105.254369) (width 0.2) (layer "B.Cu") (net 6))
 (segment (start 165.7 149.0225) (end 166.65 149.0225) (width 0.2) (layer "F.Cu") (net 4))
 (segment (start 169.75 92.9) (end 169.75 90.23) (width 0.2) (layer "F.Cu") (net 4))
 (segment (start 172.35 142.85) (end 170.55 141.05) (width 0.2) (layer "F.Cu") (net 4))
 (segment (start 164.05 158.1975) (end 172.35 158.1975) (width 0.2) (layer "F.Cu") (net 4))
 (segment (start 167.701 148.9215) (end 167.6 149.0225) (width 0.2) (layer "F.Cu") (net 4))
 (segment (start 172.35 144.4475) (end 172.35 142.85) (width 0.2) (layer "F.Cu") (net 4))
 (segment (start 164.05 144.4475) (end 164.05 147.3725) (width 0.2) (layer "F.Cu") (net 4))
 (segment (start 164.55 171.35) (end 171.05 171.35) (width 0.2) (layer "F.Cu") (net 4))
 (segment (start 167.701 143.751) (end 167.701 148.9215) (width 0.2) (layer "F.Cu") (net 4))
 (segment (start 167.6 149.0225) (end 166.65 149.0225) (width 0.2) (layer "F.Cu") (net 4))
 (segment (start 170.55 141.05) (end 170.3 141.3) (width 0.2) (layer "F.Cu") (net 4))
 (segment (start 176.301 132.901) (end 174.7 131.3) (width 0.2) (layer "F.Cu") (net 4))
 (segment (start 176.2985 158.1975) (end 176.301 158.2) (width 0.2) (layer "F.Cu") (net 4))
 (segment (start 158.3 128.1) (end 158.3 104.807985) (width 0.2) (layer "F.Cu") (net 4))
 (segment (start 176.301 166.099) (end 171.05 171.35) (width 0.2) (layer "F.Cu") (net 4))
 (segment (start 164.05 147.3725) (end 165.7 149.0225) (width 0.2) (layer "F.Cu") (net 4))
 (segment (start 158.3 104.807985) (end 160.393616 102.714369) (width 0.2) (layer "F.Cu") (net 4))
 (segment (start 176.301 158.2) (end 176.301 166.099) (width 0.2) (layer "F.Cu") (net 4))
 (segment (start 176.301 144.5) (end 176.301 158.2) (width 0.2) (layer "F.Cu") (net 4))
 (segment (start 165.25 141.3) (end 167.701 143.751) (width 0.2) (layer "F.Cu") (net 4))
 (segment (start 170.3 141.3) (end 165.25 141.3) (width 0.2) (layer "F.Cu") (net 4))
 (segment (start 176.301 144.5) (end 176.301 132.901) (width 0.2) (layer "F.Cu") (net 4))
 (segment (start 173.524 88.924) (end 174.675 90.075) (width 0.2) (layer "F.Cu") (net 4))
 (segment (start 172.35 158.1975) (end 176.2985 158.1975) (width 0.2) (layer "F.Cu") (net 4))
 (segment (start 169.75 90.23) (end 169.595 90.075) (width 0.2) (layer "F.Cu") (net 4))
 (segment (start 159.916856 121.645369) (end 160.870376 121.645369) (width 0.2) (layer "B.Cu") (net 4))
 (segment (start 172.94 88.34) (end 167.86 88.34) (width 0.2) (layer "B.Cu") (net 4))
 (segment (start 176.301 137.66516) (end 175.98516 137.981) (width 0.2) (layer "B.Cu") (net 4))
 (segment (start 162.379247 104.7) (end 160.393616 102.714369) (width 0.2) (layer "B.Cu") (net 4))
 (segment (start 160.870376 121.645369) (end 161.544616 120.971129) (width 0.2) (layer "B.Cu") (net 4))
 (segment (start 167.86 88.34) (end 167.642 88.122) (width 0.2) (layer "B.Cu") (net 4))
 (segment (start 174.675 90.075) (end 172.94 88.34) (width 0.2) (layer "B.Cu") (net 4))
 (segment (start 173.41484 137.981) (end 162.5 127.06616) (width 0.2) (layer "B.Cu") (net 4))
 (segment (start 169.595 90.075) (end 167.86 88.34) (width 0.2) (layer "B.Cu") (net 4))
 (segment (start 176.301 132.901) (end 176.301 137.66516) (width 0.2) (layer "B.Cu") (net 4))
 (segment (start 161.544616 120.971129) (end 161.544616 103.865369) (width 0.2) (layer "B.Cu") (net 4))
 (segment (start 157.5 119.228513) (end 159.916856 121.645369) (width 0.2) (layer "B.Cu") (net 4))
 (segment (start 160.4918 88.122) (end 157.5 91.1138) (width 0.2) (layer "B.Cu") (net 4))
 (segment (start 174.7 131.3) (end 176.301 132.901) (width 0.2) (layer "B.Cu") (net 4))
 (segment (start 162.5 127.06616) (end 162.5 104.7) (width 0.2) (layer "B.Cu") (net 4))
 (segment (start 161.544616 103.865369) (end 160.393616 102.714369) (width 0.2) (layer "B.Cu") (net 4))
 (segment (start 167.642 88.122) (end 160.4918 88.122) (width 0.2) (layer "B.Cu") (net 4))
 (segment (start 162.5 104.7) (end 162.379247 104.7) (width 0.2) (layer "B.Cu") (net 4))
 (segment (start 175.98516 137.981) (end 173.41484 137.981) (width 0.2) (layer "B.Cu") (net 4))
 (segment (start 157.5 91.1138) (end 157.5 119.228513) (width 0.2) (layer "B.Cu") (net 4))
 (segment (start 160.84 128.1) (end 160.84 136.2725) (width 0.2) (layer "F.Cu") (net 2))
 (segment (start 160.84 136.2725) (end 160.8125 136.3) (width 0.2) (layer "F.Cu") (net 2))
 (segment (start 161.474369 100.174369) (end 160.393616 100.174369) (width 0.2) (layer "B.Cu") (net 5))
 (segment (start 163.4 125.08) (end 163.4 102.1) (width 0.2) (layer "B.Cu") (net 5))
 (segment (start 174.7 136.38) (end 163.4 125.08) (width 0.2) (layer "B.Cu") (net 5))
 (segment (start 163.4 102.1) (end 161.474369 100.174369) (width 0.2) (layer "B.Cu") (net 5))
 (segment (start 160.6579 88.523) (end 157.901 91.2799) (width 0.2) (layer "B.Cu") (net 12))
 (segment (start 167.055 90.075) (end 165.503 88.523) (width 0.2) (layer "B.Cu") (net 12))
 (segment (start 157.901 118.001753) (end 160.393616 120.494369) (width 0.2) (layer "B.Cu") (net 12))
 (segment (start 165.503 88.523) (end 160.6579 88.523) (width 0.2) (layer "B.Cu") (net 12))
 (segment (start 157.901 91.2799) (end 157.901 118.001753) (width 0.2) (layer "B.Cu") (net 12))
 (segment (start 164.515 90.075) (end 163.364 88.924) (width 0.2) (layer "B.Cu") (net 11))
 (segment (start 160.824 88.924) (end 158.302 91.446) (width 0.2) (layer "B.Cu") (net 11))
 (segment (start 158.302 115.862753) (end 160.393616 117.954369) (width 0.2) (layer "B.Cu") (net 11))
 (segment (start 163.364 88.924) (end 160.824 88.924) (width 0.2) (layer "B.Cu") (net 11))
 (segment (start 158.302 91.446) (end 158.302 115.862753) (width 0.2) (layer "B.Cu") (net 11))
 (segment (start 161.975 90.075) (end 158.703 93.347) (width 0.2) (layer "B.Cu") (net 10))
 (segment (start 158.703 93.347) (end 158.703 113.723753) (width 0.2) (layer "B.Cu") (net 10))
 (segment (start 158.703 113.723753) (end 160.393616 115.414369) (width 0.2) (layer "B.Cu") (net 10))
 (segment (start 155.3 136.3) (end 155.3 98.3329) (width 0.2) (layer "F.Cu") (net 18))
 (segment (start 176.820353 108.479647) (end 176.25 109.05) (width 0.2) (layer "F.Cu") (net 18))
 (segment (start 161.45 142.45) (end 155.3 136.3) (width 0.2) (layer "F.Cu") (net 18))
 (segment (start 176.25 109.05) (end 175.15 109.05) (width 0.2) (layer "F.Cu") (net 18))
 (segment (start 174.518353 109.681647) (end 174.518353 111.752273) (width 0.2) (layer "F.Cu") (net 18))
 (segment (start 166.65 153.4225) (end 166.101 153.4225) (width 0.2) (layer "F.Cu") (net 18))
 (segment (start 174.518353 111.752273) (end 175.669353 112.903273) (width 0.2) (layer "F.Cu") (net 18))
 (segment (start 176.820353 104.806513) (end 176.820353 108.479647) (width 0.2) (layer "F.Cu") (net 18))
 (segment (start 175.085453 104.132273) (end 176.146113 104.132273) (width 0.2) (layer "F.Cu") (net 18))
 (segment (start 157.4339 96.199) (end 167.15218 96.199) (width 0.2) (layer "F.Cu") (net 18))
 (segment (start 176.146113 104.132273) (end 176.820353 104.806513) (width 0.2) (layer "F.Cu") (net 18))
 (segment (start 161.45 148.7715) (end 161.45 142.45) (width 0.2) (layer "F.Cu") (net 18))
 (segment (start 155.3 98.3329) (end 157.4339 96.199) (width 0.2) (layer "F.Cu") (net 18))
 (segment (start 175.15 109.05) (end 174.518353 109.681647) (width 0.2) (layer "F.Cu") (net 18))
 (segment (start 166.101 153.4225) (end 161.45 148.7715) (width 0.2) (layer "F.Cu") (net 18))
 (segment (start 167.15218 96.199) (end 175.085453 104.132273) (width 0.2) (layer "F.Cu") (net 18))
 (segment (start 179.3 158.6) (end 179.3 121.61392) (width 0.2) (layer "B.Cu") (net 3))
 (segment (start 179.3 121.61392) (end 175.669353 117.983273) (width 0.2) (layer "B.Cu") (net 3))
 (segment (start 171.05 166.85) (end 179.3 158.6) (width 0.2) (layer "B.Cu") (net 3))
 (segment (start 164.55 166.85) (end 171.05 166.85) (width 0.2) (layer "B.Cu") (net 3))
 (segment (start 175.669353 122.941807) (end 175.669353 120.523273) (width 0.2) (layer "F.Cu") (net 1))
 (segment (start 161.31016 137.301) (end 175.669353 122.941807) (width 0.2) (layer "F.Cu") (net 1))
 (segment (start 158.9875 136.3) (end 159.9885 137.301) (width 0.2) (layer "F.Cu") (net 1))
 (segment (start 159.9885 137.301) (end 161.31016 137.301) (width 0.2) (layer "F.Cu") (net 1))
 (segment (start 176.752273 111.752273) (end 179.6 114.6) (width 0.2) (layer "F.Cu") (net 17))
 (segment (start 179.6 114.6) (end 179.6 123.95) (width 0.2) (layer "F.Cu") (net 17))
 (segment (start 179.6 123.95) (end 167.4 136.15) (width 0.2) (layer "F.Cu") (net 17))
 (segment (start 176.752273 111.446193) (end 176.752273 111.752273) (width 0.2) (layer "F.Cu") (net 17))
 (segment (start 175.669353 110.363273) (end 176.752273 111.446193) (width 0.2) (layer "F.Cu") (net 17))
 (segment (start 167.6 152.3225) (end 166.65 152.3225) (width 0.2) (layer "F.Cu") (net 17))
 (segment (start 167.4 136.65) (end 175 144.25) (width 0.2) (layer "F.Cu") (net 17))
 (segment (start 175 144.25) (end 175 144.9225) (width 0.2) (layer "F.Cu") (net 17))
 (segment (start 167.4 136.15) (end 167.4 136.65) (width 0.2) (layer "F.Cu") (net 17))
 (segment (start 175 144.9225) (end 167.6 152.3225) (width 0.2) (layer "F.Cu") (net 17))
 (segment (start 162.4602 142.326) (end 156.201 136.0668) (width 0.2) (layer "F.Cu") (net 16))
 (segment (start 166.65 147.9225) (end 165.7 147.9225) (width 0.2) (layer "F.Cu") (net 16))
 (segment (start 156.201 98.599) (end 157.799 97.001) (width 0.2) (layer "F.Cu") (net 16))
 (segment (start 165.351 142.326) (end 162.4602 142.326) (width 0.2) (layer "F.Cu") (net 16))
 (segment (start 165.7 147.9225) (end 165.351 147.5735) (width 0.2) (layer "F.Cu") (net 16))
 (segment (start 166.75 101.4) (end 173.173273 107.823273) (width 0.2) (layer "F.Cu") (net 16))
 (segment (start 165.351 147.5735) (end 165.351 142.326) (width 0.2) (layer "F.Cu") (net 16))
 (segment (start 156.201 136.0668) (end 156.201 98.599) (width 0.2) (layer "F.Cu") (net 16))
 (segment (start 173.173273 107.823273) (end 175.669353 107.823273) (width 0.2) (layer "F.Cu") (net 16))
 (segment (start 157.799 97.001) (end 166.75 97.001) (width 0.2) (layer "F.Cu") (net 16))
 (segment (start 166.75 97.001) (end 166.75 101.4) (width 0.2) (layer "F.Cu") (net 16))
 (segment (start 157.6 96.6) (end 166.98608 96.6) (width 0.2) (layer "F.Cu") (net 15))
 (segment (start 161.851 142.55) (end 161.851 142.2839) (width 0.2) (layer "F.Cu") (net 15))
 (segment (start 155.8 136.2329) (end 155.8 98.4) (width 0.2) (layer "F.Cu") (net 15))
 (segment (start 165.7 150.1225) (end 161.851 146.2735) (width 0.2) (layer "F.Cu") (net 15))
 (segment (start 166.65 150.1225) (end 165.7 150.1225) (width 0.2) (layer "F.Cu") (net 15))
 (segment (start 161.851 142.2839) (end 155.8 136.2329) (width 0.2) (layer "F.Cu") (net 15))
 (segment (start 161.851 146.2735) (end 161.851 142.5799) (width 0.2) (layer "F.Cu") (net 15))
 (segment (start 155.8 98.4) (end 157.6 96.6) (width 0.2) (layer "F.Cu") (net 15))
 (segment (start 166.98608 96.6) (end 175.669353 105.283273) (width 0.2) (layer "F.Cu") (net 15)))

